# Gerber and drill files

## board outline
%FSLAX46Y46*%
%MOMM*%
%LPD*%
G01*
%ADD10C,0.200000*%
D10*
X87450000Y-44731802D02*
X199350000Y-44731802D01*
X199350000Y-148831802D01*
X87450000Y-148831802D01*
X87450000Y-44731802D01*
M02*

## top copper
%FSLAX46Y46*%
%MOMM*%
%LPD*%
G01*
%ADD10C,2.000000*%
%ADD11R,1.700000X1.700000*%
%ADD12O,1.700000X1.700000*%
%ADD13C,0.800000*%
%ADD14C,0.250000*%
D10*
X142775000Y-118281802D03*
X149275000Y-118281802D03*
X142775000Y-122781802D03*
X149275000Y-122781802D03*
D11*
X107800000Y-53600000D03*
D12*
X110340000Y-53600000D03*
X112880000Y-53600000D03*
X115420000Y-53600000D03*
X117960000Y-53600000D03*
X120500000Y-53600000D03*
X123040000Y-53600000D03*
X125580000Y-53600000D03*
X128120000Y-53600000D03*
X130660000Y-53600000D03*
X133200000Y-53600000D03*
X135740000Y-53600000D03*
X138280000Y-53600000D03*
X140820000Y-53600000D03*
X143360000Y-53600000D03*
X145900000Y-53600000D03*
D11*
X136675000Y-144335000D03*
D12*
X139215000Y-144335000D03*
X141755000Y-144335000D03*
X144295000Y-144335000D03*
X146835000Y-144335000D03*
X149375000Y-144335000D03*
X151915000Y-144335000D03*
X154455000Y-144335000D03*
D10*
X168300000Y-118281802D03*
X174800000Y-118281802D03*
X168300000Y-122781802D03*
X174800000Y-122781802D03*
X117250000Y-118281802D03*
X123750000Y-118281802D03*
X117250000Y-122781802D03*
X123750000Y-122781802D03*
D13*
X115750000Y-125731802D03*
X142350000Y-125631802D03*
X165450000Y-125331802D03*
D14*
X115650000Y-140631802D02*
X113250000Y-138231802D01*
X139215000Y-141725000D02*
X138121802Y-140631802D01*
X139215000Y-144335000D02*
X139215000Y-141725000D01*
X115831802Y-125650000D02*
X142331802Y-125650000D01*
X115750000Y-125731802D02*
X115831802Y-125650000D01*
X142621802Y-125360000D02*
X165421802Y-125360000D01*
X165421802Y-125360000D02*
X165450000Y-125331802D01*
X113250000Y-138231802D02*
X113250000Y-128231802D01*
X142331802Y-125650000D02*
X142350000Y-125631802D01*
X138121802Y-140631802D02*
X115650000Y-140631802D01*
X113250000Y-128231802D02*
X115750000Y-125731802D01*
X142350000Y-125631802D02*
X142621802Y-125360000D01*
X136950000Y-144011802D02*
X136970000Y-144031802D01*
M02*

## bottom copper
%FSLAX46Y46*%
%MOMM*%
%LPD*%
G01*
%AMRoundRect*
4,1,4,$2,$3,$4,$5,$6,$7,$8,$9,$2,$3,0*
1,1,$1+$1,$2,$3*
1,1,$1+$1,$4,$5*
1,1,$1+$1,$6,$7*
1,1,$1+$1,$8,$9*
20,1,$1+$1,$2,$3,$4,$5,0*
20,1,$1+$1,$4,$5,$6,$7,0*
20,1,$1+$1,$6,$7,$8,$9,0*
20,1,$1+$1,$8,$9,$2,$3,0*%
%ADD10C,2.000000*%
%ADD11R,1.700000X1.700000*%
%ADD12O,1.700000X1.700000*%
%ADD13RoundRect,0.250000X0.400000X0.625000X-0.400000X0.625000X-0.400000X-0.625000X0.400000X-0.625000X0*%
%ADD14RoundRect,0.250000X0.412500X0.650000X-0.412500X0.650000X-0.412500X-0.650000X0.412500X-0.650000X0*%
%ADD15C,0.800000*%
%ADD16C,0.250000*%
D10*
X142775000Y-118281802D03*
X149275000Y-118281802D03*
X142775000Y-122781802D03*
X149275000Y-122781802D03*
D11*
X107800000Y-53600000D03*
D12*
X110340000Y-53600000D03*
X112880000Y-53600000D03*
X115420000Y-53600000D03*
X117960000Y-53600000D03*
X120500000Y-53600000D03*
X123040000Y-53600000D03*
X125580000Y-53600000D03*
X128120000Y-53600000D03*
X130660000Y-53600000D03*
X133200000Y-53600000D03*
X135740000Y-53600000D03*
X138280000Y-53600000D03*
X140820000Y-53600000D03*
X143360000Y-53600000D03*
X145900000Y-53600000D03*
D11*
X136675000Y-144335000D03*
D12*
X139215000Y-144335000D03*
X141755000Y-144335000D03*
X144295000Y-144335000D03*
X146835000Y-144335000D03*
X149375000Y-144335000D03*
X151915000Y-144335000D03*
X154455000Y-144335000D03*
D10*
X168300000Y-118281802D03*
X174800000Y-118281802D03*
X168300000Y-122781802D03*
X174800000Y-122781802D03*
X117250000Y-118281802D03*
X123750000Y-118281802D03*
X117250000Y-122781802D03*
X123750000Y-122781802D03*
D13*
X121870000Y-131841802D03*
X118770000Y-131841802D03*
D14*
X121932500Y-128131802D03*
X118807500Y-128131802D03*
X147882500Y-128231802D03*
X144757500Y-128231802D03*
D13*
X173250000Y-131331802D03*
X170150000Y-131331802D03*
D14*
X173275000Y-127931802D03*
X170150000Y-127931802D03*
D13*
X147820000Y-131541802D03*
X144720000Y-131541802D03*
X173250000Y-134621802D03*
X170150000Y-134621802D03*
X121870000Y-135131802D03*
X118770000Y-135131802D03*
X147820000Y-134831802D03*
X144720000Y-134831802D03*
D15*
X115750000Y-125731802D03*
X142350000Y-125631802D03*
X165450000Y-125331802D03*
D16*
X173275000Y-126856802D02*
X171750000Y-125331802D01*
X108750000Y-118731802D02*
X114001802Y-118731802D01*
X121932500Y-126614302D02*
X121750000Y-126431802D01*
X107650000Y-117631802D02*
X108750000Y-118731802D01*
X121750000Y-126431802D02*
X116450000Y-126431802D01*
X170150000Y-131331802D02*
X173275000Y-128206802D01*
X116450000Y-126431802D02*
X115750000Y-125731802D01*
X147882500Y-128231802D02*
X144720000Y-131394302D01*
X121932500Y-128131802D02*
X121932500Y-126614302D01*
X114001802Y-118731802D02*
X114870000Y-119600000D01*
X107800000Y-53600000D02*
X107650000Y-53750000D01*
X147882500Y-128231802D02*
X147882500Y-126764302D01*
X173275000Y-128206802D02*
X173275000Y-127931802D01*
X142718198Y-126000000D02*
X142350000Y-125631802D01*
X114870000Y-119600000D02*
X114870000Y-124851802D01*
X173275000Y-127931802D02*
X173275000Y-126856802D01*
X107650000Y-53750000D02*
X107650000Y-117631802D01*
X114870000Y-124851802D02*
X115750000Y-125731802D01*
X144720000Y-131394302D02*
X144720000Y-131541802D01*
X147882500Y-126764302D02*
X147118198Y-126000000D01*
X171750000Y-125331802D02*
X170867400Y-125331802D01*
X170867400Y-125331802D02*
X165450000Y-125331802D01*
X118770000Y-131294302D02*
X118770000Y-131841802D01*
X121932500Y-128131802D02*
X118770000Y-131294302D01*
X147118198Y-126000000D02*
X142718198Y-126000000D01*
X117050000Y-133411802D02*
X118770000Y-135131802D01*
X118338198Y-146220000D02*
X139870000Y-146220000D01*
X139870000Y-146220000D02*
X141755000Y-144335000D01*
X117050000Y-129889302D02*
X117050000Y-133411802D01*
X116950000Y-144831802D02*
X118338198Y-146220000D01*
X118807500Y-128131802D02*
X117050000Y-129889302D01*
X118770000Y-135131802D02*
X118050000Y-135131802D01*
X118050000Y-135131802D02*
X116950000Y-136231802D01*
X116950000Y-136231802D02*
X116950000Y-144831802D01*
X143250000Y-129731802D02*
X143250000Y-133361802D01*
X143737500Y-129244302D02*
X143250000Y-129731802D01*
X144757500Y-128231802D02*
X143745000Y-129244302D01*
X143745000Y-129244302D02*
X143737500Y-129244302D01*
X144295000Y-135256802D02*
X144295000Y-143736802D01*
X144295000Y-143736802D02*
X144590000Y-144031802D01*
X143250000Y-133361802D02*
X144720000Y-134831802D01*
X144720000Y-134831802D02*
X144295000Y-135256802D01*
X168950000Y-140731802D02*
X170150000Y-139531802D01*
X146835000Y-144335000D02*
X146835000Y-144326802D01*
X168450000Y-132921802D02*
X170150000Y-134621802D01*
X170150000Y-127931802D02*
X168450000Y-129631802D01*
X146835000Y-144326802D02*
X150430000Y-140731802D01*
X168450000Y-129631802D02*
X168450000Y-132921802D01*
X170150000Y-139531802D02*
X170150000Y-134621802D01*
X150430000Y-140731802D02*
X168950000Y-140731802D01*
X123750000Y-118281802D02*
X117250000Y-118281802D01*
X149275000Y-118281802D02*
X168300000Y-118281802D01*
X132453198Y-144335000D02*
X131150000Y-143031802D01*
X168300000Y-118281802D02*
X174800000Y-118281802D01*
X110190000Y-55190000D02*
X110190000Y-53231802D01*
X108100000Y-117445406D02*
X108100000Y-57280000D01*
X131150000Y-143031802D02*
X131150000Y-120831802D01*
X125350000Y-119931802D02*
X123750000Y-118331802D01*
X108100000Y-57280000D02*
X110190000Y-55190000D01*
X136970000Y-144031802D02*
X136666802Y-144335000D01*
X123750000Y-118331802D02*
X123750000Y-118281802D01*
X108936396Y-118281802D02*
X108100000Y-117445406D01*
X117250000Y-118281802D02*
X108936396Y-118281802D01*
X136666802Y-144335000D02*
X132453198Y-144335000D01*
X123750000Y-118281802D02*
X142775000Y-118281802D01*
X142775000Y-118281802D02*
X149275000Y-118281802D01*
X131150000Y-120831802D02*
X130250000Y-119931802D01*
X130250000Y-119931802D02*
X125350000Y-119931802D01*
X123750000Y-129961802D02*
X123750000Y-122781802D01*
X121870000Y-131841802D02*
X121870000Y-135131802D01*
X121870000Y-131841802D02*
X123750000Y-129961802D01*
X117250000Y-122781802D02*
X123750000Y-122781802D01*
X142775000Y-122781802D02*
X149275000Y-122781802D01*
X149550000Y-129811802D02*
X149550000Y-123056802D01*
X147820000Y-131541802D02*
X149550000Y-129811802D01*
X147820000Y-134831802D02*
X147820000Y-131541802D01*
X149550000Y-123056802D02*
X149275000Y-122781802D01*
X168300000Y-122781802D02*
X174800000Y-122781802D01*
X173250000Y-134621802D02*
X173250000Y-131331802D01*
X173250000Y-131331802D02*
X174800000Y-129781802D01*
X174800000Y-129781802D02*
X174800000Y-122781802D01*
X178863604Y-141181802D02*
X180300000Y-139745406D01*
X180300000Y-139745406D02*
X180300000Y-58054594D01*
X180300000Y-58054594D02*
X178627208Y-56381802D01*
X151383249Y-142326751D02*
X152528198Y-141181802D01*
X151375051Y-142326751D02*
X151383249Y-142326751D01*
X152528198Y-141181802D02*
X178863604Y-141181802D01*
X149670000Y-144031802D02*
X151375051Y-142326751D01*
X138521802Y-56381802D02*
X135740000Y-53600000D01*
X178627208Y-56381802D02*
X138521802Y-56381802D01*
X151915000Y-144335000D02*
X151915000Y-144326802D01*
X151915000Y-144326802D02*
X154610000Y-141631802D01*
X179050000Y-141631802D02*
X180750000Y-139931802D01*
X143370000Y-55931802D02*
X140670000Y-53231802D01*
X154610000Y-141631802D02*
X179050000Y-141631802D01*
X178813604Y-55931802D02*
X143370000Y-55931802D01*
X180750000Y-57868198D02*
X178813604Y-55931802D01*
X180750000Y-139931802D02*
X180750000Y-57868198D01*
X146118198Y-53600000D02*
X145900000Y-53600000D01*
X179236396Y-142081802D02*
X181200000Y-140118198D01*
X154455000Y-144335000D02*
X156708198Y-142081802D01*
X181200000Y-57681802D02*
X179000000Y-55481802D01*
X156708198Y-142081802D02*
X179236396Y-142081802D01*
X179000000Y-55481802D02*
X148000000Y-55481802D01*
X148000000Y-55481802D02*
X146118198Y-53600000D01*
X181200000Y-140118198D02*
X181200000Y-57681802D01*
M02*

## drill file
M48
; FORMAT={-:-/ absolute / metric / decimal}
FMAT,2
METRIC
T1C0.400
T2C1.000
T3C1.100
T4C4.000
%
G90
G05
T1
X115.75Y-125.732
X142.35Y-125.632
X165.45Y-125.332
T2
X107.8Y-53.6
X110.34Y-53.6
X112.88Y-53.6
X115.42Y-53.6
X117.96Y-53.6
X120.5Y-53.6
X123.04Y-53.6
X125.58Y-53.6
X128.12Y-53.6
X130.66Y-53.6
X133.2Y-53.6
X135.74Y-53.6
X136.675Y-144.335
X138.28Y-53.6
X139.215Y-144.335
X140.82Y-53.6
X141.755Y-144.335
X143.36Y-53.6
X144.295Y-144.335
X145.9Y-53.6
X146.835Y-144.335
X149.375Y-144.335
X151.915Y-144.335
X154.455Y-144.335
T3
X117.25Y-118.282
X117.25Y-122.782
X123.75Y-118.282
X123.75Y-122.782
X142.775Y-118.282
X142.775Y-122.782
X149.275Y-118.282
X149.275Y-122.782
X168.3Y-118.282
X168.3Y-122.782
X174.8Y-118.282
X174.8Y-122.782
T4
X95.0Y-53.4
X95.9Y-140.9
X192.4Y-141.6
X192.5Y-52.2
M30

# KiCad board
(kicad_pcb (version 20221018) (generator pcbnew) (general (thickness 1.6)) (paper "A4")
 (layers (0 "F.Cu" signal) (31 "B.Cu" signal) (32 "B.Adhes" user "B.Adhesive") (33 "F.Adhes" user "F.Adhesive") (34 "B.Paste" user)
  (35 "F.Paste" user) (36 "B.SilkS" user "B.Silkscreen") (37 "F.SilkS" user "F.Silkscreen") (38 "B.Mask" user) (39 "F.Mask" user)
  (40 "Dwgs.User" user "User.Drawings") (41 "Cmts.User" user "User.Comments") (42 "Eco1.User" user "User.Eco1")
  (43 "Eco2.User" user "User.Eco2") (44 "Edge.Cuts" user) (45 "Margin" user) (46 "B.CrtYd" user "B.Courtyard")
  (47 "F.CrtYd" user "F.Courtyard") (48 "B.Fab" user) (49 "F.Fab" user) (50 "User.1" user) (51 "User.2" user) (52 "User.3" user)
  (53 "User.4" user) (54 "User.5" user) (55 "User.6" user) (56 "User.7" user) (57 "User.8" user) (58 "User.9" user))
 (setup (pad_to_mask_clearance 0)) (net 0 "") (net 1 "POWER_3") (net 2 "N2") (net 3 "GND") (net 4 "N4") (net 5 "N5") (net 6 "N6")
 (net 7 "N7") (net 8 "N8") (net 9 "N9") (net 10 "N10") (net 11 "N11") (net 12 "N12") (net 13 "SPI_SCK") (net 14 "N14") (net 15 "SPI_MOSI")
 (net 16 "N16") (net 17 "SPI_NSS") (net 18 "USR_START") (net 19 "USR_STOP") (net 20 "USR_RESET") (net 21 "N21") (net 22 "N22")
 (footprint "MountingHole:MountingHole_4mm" (layer "F.Cu") (at 192.4 141.6)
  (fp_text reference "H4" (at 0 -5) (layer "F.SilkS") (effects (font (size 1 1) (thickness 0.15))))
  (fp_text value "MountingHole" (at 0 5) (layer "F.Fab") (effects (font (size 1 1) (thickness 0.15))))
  (pad "" np_thru_hole circle (at 0 0) (size 4 4) (drill 4) (layers "*.Cu" "*.Mask")))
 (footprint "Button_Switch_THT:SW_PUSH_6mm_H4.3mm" (layer "F.Cu") (at 142.775 118.281802)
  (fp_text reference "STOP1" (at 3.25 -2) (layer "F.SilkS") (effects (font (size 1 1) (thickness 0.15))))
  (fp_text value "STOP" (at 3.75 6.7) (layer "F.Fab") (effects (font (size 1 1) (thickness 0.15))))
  (pad "1" thru_hole circle (at 0 0 90) (size 2 2) (drill 1.1) (layers "*.Cu" "*.Mask") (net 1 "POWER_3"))
  (pad "1" thru_hole circle (at 6.5 0 90) (size 2 2) (drill 1.1) (layers "*.Cu" "*.Mask") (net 1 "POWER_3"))
  (pad "2" thru_hole circle (at 0 4.5 90) (size 2 2) (drill 1.1) (layers "*.Cu" "*.Mask") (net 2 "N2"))
  (pad "2" thru_hole circle (at 6.5 4.5 90) (size 2 2) (drill 1.1) (layers "*.Cu" "*.Mask") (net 2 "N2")))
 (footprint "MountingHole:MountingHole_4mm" (layer "F.Cu") (at 95.9 140.9)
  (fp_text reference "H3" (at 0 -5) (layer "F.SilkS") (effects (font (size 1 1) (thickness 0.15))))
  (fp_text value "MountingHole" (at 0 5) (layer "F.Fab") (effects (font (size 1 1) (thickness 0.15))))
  (pad "" np_thru_hole circle (at 0 0) (size 4 4) (drill 4) (layers "*.Cu" "*.Mask")))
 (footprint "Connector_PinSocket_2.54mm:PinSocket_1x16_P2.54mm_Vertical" (layer "F.Cu") (at 107.8 53.6 90)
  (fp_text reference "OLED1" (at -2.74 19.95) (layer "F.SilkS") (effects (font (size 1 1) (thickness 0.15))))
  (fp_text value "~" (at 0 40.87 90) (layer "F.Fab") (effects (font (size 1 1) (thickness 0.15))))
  (pad "1" thru_hole rect (at 0 0 90) (size 1.7 1.7) (drill 1) (layers "*.Cu" "*.Mask") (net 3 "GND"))
  (pad "2" thru_hole oval (at 0 2.54 90) (size 1.7 1.7) (drill 1) (layers "*.Cu" "*.Mask") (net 1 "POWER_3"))
  (pad "3" thru_hole oval (at 0 5.08 90) (size 1.7 1.7) (drill 1) (layers "*.Cu" "*.Mask") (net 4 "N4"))
  (pad "4" thru_hole oval (at 0 7.62 90) (size 1.7 1.7) (drill 1) (layers "*.Cu" "*.Mask") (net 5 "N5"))
  (pad "5" thru_hole oval (at 0 10.16 90) (size 1.7 1.7) (drill 1) (layers "*.Cu" "*.Mask") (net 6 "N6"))
  (pad "6" thru_hole oval (at 0 12.7 90) (size 1.7 1.7) (drill 1) (layers "*.Cu" "*.Mask") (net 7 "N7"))
  (pad "7" thru_hole oval (at 0 15.24 90) (size 1.7 1.7) (drill 1) (layers "*.Cu" "*.Mask") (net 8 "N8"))
  (pad "8" thru_hole oval (at 0 17.78 90) (size 1.7 1.7) (drill 1) (layers "*.Cu" "*.Mask") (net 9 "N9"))
  (pad "9" thru_hole oval (at 0 20.32 90) (size 1.7 1.7) (drill 1) (layers "*.Cu" "*.Mask") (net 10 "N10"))
  (pad "10" thru_hole oval (at 0 22.86 90) (size 1.7 1.7) (drill 1) (layers "*.Cu" "*.Mask") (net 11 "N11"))
  (pad "11" thru_hole oval (at 0 25.4 90) (size 1.7 1.7) (drill 1) (layers "*.Cu" "*.Mask") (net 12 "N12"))
  (pad "12" thru_hole oval (at 0 27.94 90) (size 1.7 1.7) (drill 1) (layers "*.Cu" "*.Mask") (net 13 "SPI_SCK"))
  (pad "13" thru_hole oval (at 0 30.48 90) (size 1.7 1.7) (drill 1) (layers "*.Cu" "*.Mask") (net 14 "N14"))
  (pad "14" thru_hole oval (at 0 33.02 90) (size 1.7 1.7) (drill 1) (layers "*.Cu" "*.Mask") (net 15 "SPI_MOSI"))
  (pad "15" thru_hole oval (at 0 35.56 90) (size 1.7 1.7) (drill 1) (layers "*.Cu" "*.Mask") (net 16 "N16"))
  (pad "16" thru_hole oval (at 0 38.1 90) (size 1.7 1.7) (drill 1) (layers "*.Cu" "*.Mask") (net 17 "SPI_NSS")))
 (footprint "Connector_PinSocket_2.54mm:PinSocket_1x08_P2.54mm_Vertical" (layer "F.Cu") (at 136.675 144.335 90)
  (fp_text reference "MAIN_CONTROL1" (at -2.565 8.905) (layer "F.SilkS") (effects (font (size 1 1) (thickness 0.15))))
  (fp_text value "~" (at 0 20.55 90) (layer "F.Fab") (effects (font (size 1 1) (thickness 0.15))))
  (pad "1" thru_hole rect (at 0 0 90) (size 1.7 1.7) (drill 1) (layers "*.Cu" "*.Mask") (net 1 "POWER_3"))
  (pad "2" thru_hole oval (at 0 2.54 90) (size 1.7 1.7) (drill 1) (layers "*.Cu" "*.Mask") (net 3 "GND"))
  (pad "3" thru_hole oval (at 0 5.08 90) (size 1.7 1.7) (drill 1) (layers "*.Cu" "*.Mask") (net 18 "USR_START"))
  (pad "4" thru_hole oval (at 0 7.62 90) (size 1.7 1.7) (drill 1) (layers "*.Cu" "*.Mask") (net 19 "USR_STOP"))
  (pad "5" thru_hole oval (at 0 10.16 90) (size 1.7 1.7) (drill 1) (layers "*.Cu" "*.Mask") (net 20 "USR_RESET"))
  (pad "6" thru_hole oval (at 0 12.7 90) (size 1.7 1.7) (drill 1) (layers "*.Cu" "*.Mask") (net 13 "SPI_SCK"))
  (pad "7" thru_hole oval (at 0 15.24 90) (size 1.7 1.7) (drill 1) (layers "*.Cu" "*.Mask") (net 15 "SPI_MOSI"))
  (pad "8" thru_hole oval (at 0 17.78 90) (size 1.7 1.7) (drill 1) (layers "*.Cu" "*.Mask") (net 17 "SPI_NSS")))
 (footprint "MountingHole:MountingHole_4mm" (layer "F.Cu") (at 192.5 52.2)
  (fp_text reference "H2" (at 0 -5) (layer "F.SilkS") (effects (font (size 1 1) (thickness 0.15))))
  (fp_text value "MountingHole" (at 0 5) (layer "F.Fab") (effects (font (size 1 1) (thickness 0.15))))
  (pad "" np_thru_hole circle (at 0 0) (size 4 4) (drill 4) (layers "*.Cu" "*.Mask")))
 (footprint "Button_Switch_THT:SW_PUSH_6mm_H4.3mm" (layer "F.Cu") (at 168.3 118.281802)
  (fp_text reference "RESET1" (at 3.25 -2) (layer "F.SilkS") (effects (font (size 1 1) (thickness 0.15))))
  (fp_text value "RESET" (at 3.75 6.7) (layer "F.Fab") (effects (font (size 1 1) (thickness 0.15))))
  (pad "1" thru_hole circle (at 0 0 90) (size 2 2) (drill 1.1) (layers "*.Cu" "*.Mask") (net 1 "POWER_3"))
  (pad "1" thru_hole circle (at 6.5 0 90) (size 2 2) (drill 1.1) (layers "*.Cu" "*.Mask") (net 1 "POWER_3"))
  (pad "2" thru_hole circle (at 0 4.5 90) (size 2 2) (drill 1.1) (layers "*.Cu" "*.Mask") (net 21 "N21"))
  (pad "2" thru_hole circle (at 6.5 4.5 90) (size 2 2) (drill 1.1) (layers "*.Cu" "*.Mask") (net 21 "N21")))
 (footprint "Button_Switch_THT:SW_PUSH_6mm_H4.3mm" (layer "F.Cu") (at 117.25 118.281802)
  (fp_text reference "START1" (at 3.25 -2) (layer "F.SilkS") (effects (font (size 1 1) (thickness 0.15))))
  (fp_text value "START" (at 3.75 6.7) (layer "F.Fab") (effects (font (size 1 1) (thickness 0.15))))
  (pad "1" thru_hole circle (at 0 0 90) (size 2 2) (drill 1.1) (layers "*.Cu" "*.Mask") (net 1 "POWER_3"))
  (pad "1" thru_hole circle (at 6.5 0 90) (size 2 2) (drill 1.1) (layers "*.Cu" "*.Mask") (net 1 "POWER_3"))
  (pad "2" thru_hole circle (at 0 4.5 90) (size 2 2) (drill 1.1) (layers "*.Cu" "*.Mask") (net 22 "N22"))
  (pad "2" thru_hole circle (at 6.5 4.5 90) (size 2 2) (drill 1.1) (layers "*.Cu" "*.Mask") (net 22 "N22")))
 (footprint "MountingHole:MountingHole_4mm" (layer "F.Cu") (at 95 53.4)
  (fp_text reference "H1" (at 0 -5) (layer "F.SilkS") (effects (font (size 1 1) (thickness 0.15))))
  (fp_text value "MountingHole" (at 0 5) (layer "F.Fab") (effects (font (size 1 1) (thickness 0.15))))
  (pad "" np_thru_hole circle (at 0 0) (size 4 4) (drill 4) (layers "*.Cu" "*.Mask")))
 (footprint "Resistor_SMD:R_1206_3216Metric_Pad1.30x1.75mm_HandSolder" (layer "B.Cu") (at 120.32 131.841802 180)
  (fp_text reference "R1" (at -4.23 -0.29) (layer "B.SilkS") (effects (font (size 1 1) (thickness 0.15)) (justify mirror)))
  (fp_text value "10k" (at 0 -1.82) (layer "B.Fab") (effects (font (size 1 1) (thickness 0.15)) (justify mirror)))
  (pad "1" smd roundrect (at -1.55 0 180) (size 1.3 1.75) (layers "B.Cu" "B.Paste" "B.Mask") (roundrect_rratio 0.192308) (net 22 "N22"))
  (pad "2" smd roundrect (at 1.55 0 180) (size 1.3 1.75) (layers "B.Cu" "B.Paste" "B.Mask") (roundrect_rratio 0.192308) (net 3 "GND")))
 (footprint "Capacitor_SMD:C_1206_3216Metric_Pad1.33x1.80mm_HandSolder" (layer "B.Cu") (at 120.37 128.131802 180)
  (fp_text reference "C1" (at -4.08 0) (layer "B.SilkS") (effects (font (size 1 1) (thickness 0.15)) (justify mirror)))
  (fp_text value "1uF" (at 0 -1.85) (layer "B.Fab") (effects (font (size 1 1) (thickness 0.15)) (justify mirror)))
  (pad "1" smd roundrect (at -1.5625 0 180) (size 1.325 1.8) (layers "B.Cu" "B.Paste" "B.Mask") (roundrect_rratio 0.188679) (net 3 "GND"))
  (pad "2" smd roundrect (at 1.5625 0 180) (size 1.325 1.8) (layers "B.Cu" "B.Paste" "B.Mask") (roundrect_rratio 0.188679)
   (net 18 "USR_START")))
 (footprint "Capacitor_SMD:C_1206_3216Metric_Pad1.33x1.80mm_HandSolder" (layer "B.Cu") (at 146.32 128.231802 180)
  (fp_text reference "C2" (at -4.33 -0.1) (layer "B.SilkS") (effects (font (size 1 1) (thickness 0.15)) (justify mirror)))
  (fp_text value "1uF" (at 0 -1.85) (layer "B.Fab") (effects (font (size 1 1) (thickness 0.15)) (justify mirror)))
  (pad "1" smd roundrect (at -1.5625 0 180) (size 1.325 1.8) (layers "B.Cu" "B.Paste" "B.Mask") (roundrect_rratio 0.188679) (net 3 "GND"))
  (pad "2" smd roundrect (at 1.5625 0 180) (size 1.325 1.8) (layers "B.Cu" "B.Paste" "B.Mask") (roundrect_rratio 0.188679)
   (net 19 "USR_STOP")))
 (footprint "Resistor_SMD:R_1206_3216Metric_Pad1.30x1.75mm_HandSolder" (layer "B.Cu") (at 171.7 131.331802 180)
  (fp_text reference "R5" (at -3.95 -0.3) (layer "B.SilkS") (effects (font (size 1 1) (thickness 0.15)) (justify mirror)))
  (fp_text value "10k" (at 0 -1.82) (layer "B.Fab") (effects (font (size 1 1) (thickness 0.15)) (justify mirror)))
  (pad "1" smd roundrect (at -1.55 0 180) (size 1.3 1.75) (layers "B.Cu" "B.Paste" "B.Mask") (roundrect_rratio 0.192308) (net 21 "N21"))
  (pad "2" smd roundrect (at 1.55 0 180) (size 1.3 1.75) (layers "B.Cu" "B.Paste" "B.Mask") (roundrect_rratio 0.192308) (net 3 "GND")))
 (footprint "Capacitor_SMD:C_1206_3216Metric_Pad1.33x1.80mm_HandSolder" (layer "B.Cu") (at 171.7125 127.931802 180)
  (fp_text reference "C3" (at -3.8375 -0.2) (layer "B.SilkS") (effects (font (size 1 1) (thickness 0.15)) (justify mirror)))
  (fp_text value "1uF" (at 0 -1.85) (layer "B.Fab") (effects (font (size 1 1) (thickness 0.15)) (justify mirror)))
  (pad "1" smd roundrect (at -1.5625 0 180) (size 1.325 1.8) (layers "B.Cu" "B.Paste" "B.Mask") (roundrect_rratio 0.188679) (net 3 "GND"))
  (pad "2" smd roundrect (at 1.5625 0 180) (size 1.325 1.8) (layers "B.Cu" "B.Paste" "B.Mask") (roundrect_rratio 0.188679)
   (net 20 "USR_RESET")))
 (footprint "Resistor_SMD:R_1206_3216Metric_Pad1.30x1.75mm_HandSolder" (layer "B.Cu") (at 146.27 131.541802 180)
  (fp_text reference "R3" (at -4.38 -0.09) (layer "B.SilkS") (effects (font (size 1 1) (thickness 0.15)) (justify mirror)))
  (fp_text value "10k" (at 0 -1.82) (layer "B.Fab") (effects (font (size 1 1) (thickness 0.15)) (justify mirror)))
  (pad "1" smd roundrect (at -1.55 0 180) (size 1.3 1.75) (layers "B.Cu" "B.Paste" "B.Mask") (roundrect_rratio 0.192308) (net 2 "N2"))
  (pad "2" smd roundrect (at 1.55 0 180) (size 1.3 1.75) (layers "B.Cu" "B.Paste" "B.Mask") (roundrect_rratio 0.192308) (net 3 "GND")))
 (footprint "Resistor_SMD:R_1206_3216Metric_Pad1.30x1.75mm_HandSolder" (layer "B.Cu") (at 171.7 134.621802 180)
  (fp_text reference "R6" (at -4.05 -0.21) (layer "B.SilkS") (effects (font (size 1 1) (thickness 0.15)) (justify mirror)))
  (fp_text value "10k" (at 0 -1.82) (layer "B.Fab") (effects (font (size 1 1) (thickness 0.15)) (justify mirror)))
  (pad "1" smd roundrect (at -1.55 0 180) (size 1.3 1.75) (layers "B.Cu" "B.Paste" "B.Mask") (roundrect_rratio 0.192308) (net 21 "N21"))
  (pad "2" smd roundrect (at 1.55 0 180) (size 1.3 1.75) (layers "B.Cu" "B.Paste" "B.Mask") (roundrect_rratio 0.192308) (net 20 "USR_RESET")))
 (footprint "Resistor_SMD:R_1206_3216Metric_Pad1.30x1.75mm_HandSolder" (layer "B.Cu") (at 120.32 135.131802 180)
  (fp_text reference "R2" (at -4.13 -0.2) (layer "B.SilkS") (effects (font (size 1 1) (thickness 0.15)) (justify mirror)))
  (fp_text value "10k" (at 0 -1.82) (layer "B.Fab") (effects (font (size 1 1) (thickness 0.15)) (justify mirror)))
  (pad "1" smd roundrect (at -1.55 0 180) (size 1.3 1.75) (layers "B.Cu" "B.Paste" "B.Mask") (roundrect_rratio 0.192308) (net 22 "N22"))
  (pad "2" smd roundrect (at 1.55 0 180) (size 1.3 1.75) (layers "B.Cu" "B.Paste" "B.Mask") (roundrect_rratio 0.192308) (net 18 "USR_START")))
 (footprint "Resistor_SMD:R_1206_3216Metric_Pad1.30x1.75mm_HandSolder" (layer "B.Cu") (at 146.27 134.831802 180)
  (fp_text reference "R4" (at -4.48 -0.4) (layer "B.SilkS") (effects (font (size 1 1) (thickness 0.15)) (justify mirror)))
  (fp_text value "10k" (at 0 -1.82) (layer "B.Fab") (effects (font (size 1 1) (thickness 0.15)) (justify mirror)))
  (pad "1" smd roundrect (at -1.55 0 180) (size 1.3 1.75) (layers "B.Cu" "B.Paste" "B.Mask") (roundrect_rratio 0.192308) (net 2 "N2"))
  (pad "2" smd roundrect (at 1.55 0 180) (size 1.3 1.75) (layers "B.Cu" "B.Paste" "B.Mask") (roundrect_rratio 0.192308) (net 19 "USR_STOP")))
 (gr_rect (start 87.45 44.731802) (end 199.35 148.831802) (stroke (width 0.2) (type default)) (fill none) (layer "Edge.Cuts"))
 (segment (start 115.65 140.631802) (end 113.25 138.231802) (width 0.25) (layer "F.Cu") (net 3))
 (segment (start 139.215 141.725) (end 138.121802 140.631802) (width 0.25) (layer "F.Cu") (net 3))
 (segment (start 139.215 144.335) (end 139.215 141.725) (width 0.25) (layer "F.Cu") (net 3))
 (segment (start 115.831802 125.65) (end 142.331802 125.65) (width 0.25) (layer "F.Cu") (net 3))
 (segment (start 115.75 125.731802) (end 115.831802 125.65) (width 0.25) (layer "F.Cu") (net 3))
 (segment (start 142.621802 125.36) (end 165.421802 125.36) (width 0.25) (layer "F.Cu") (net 3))
 (segment (start 165.421802 125.36) (end 165.45 125.331802) (width 0.25) (layer "F.Cu") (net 3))
 (segment (start 113.25 138.231802) (end 113.25 128.231802) (width 0.25) (layer "F.Cu") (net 3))
 (segment (start 142.331802 125.65) (end 142.35 125.631802) (width 0.25) (layer "F.Cu") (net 3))
 (segment (start 138.121802 140.631802) (end 115.65 140.631802) (width 0.25) (layer "F.Cu") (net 3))
 (segment (start 113.25 128.231802) (end 115.75 125.731802) (width 0.25) (layer "F.Cu") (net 3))
 (segment (start 142.35 125.631802) (end 142.621802 125.36) (width 0.25) (layer "F.Cu") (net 3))
 (via (at 115.75 125.731802) (size 0.8) (drill 0.4) (layers "F.Cu" "B.Cu") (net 3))
 (via (at 142.35 125.631802) (size 0.8) (drill 0.4) (layers "F.Cu" "B.Cu") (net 3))
 (via (at 165.45 125.331802) (size 0.8) (drill 0.4) (layers "F.Cu" "B.Cu") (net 3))
 (segment (start 173.275 126.856802) (end 171.75 125.331802) (width 0.25) (layer "B.Cu") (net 3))
 (segment (start 108.75 118.731802) (end 114.001802 118.731802) (width 0.25) (layer "B.Cu") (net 3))
 (segment (start 121.9325 126.614302) (end 121.75 126.431802) (width 0.25) (layer "B.Cu") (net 3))
 (segment (start 107.65 117.631802) (end 108.75 118.731802) (width 0.25) (layer "B.Cu") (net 3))
 (segment (start 121.75 126.431802) (end 116.45 126.431802) (width 0.25) (layer "B.Cu") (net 3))
 (segment (start 170.15 131.331802) (end 173.275 128.206802) (width 0.25) (layer "B.Cu") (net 3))
 (segment (start 116.45 126.431802) (end 115.75 125.731802) (width 0.25) (layer "B.Cu") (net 3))
 (segment (start 147.8825 128.231802) (end 144.72 131.394302) (width 0.25) (layer "B.Cu") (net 3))
 (segment (start 121.9325 128.131802) (end 121.9325 126.614302) (width 0.25) (layer "B.Cu") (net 3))
 (segment (start 114.001802 118.731802) (end 114.87 119.6) (width 0.25) (layer "B.Cu") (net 3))
 (segment (start 107.8 53.6) (end 107.65 53.75) (width 0.25) (layer "B.Cu") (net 3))
 (segment (start 147.8825 128.231802) (end 147.8825 126.764302) (width 0.25) (layer "B.Cu") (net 3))
 (segment (start 173.275 128.206802) (end 173.275 127.931802) (width 0.25) (layer "B.Cu") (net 3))
 (segment (start 142.718198 126) (end 142.35 125.631802) (width 0.25) (layer "B.Cu") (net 3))
 (segment (start 114.87 119.6) (end 114.87 124.851802) (width 0.25) (layer "B.Cu") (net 3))
 (segment (start 173.275 127.931802) (end 173.275 126.856802) (width 0.25) (layer "B.Cu") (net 3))
 (segment (start 107.65 53.75) (end 107.65 117.631802) (width 0.25) (layer "B.Cu") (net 3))
 (segment (start 114.87 124.851802) (end 115.75 125.731802) (width 0.25) (layer "B.Cu") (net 3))
 (segment (start 144.72 131.394302) (end 144.72 131.541802) (width 0.25) (layer "B.Cu") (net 3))
 (segment (start 147.8825 126.764302) (end 147.118198 126) (width 0.25) (layer "B.Cu") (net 3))
 (segment (start 171.75 125.331802) (end 170.8674 125.331802) (width 0.25) (layer "B.Cu") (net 3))
 (segment (start 170.8674 125.331802) (end 165.45 125.331802) (width 0.25) (layer "B.Cu") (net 3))
 (segment (start 118.77 131.294302) (end 118.77 131.841802) (width 0.25) (layer "B.Cu") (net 3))
 (segment (start 121.9325 128.131802) (end 118.77 131.294302) (width 0.25) (layer "B.Cu") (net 3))
 (segment (start 147.118198 126) (end 142.718198 126) (width 0.25) (layer "B.Cu") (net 3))
 (segment (start 117.05 133.411802) (end 118.77 135.131802) (width 0.25) (layer "B.Cu") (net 18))
 (segment (start 118.338198 146.22) (end 139.87 146.22) (width 0.25) (layer "B.Cu") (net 18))
 (segment (start 139.87 146.22) (end 141.755 144.335) (width 0.25) (layer "B.Cu") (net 18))
 (segment (start 117.05 129.889302) (end 117.05 133.411802) (width 0.25) (layer "B.Cu") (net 18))
 (segment (start 116.95 144.831802) (end 118.338198 146.22) (width 0.25) (layer "B.Cu") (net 18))
 (segment (start 118.8075 128.131802) (end 117.05 129.889302) (width 0.25) (layer "B.Cu") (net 18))
 (segment (start 118.77 135.131802) (end 118.05 135.131802) (width 0.25) (layer "B.Cu") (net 18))
 (segment (start 118.05 135.131802) (end 116.95 136.231802) (width 0.25) (layer "B.Cu") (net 18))
 (segment (start 116.95 136.231802) (end 116.95 144.831802) (width 0.25) (layer "B.Cu") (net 18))
 (segment (start 143.25 129.731802) (end 143.25 133.361802) (width 0.25) (layer "B.Cu") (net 19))
 (segment (start 143.7375 129.244302) (end 143.25 129.731802) (width 0.25) (layer "B.Cu") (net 19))
 (segment (start 144.7575 128.231802) (end 143.745 129.244302) (width 0.25) (layer "B.Cu") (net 19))
 (segment (start 143.745 129.244302) (end 143.7375 129.244302) (width 0.25) (layer "B.Cu") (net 19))
 (segment (start 144.295 135.256802) (end 144.295 143.736802) (width 0.25) (layer "B.Cu") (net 19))
 (segment (start 144.295 143.736802) (end 144.59 144.031802) (width 0.25) (layer "B.Cu") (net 19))
 (segment (start 143.25 133.361802) (end 144.72 134.831802) (width 0.25) (layer "B.Cu") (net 19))
 (segment (start 144.72 134.831802) (end 144.295 135.256802) (width 0.25) (layer "B.Cu") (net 19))
 (segment (start 168.95 140.731802) (end 170.15 139.531802) (width 0.25) (layer "B.Cu") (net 20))
 (segment (start 146.835 144.335) (end 146.835 144.326802) (width 0.25) (layer "B.Cu") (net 20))
 (segment (start 168.45 132.921802) (end 170.15 134.621802) (width 0.25) (layer "B.Cu") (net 20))
 (segment (start 170.15 127.931802) (end 168.45 129.631802) (width 0.25) (layer "B.Cu") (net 20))
 (segment (start 146.835 144.326802) (end 150.43 140.731802) (width 0.25) (layer "B.Cu") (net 20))
 (segment (start 168.45 129.631802) (end 168.45 132.921802) (width 0.25) (layer "B.Cu") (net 20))
 (segment (start 170.15 139.531802) (end 170.15 134.621802) (width 0.25) (layer "B.Cu") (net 20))
 (segment (start 150.43 140.731802) (end 168.95 140.731802) (width 0.25) (layer "B.Cu") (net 20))
 (segment (start 136.95 144.011802) (end 136.97 144.031802) (width 0.25) (layer "F.Cu") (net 1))
 (segment (start 123.75 118.281802) (end 117.25 118.281802) (width 0.25) (layer "B.Cu") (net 1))
 (segment (start 149.275 118.281802) (end 168.3 118.281802) (width 0.25) (layer "B.Cu") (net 1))
 (segment (start 132.453198 144.335) (end 131.15 143.031802) (width 0.25) (layer "B.Cu") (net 1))
 (segment (start 168.3 118.281802) (end 174.8 118.281802) (width 0.25) (layer "B.Cu") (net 1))
 (segment (start 110.19 55.19) (end 110.19 53.231802) (width 0.25) (layer "B.Cu") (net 1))
 (segment (start 108.1 117.445406) (end 108.1 57.28) (width 0.25) (layer "B.Cu") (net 1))
 (segment (start 131.15 143.031802) (end 131.15 120.831802) (width 0.25) (layer "B.Cu") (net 1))
 (segment (start 125.35 119.931802) (end 123.75 118.331802) (width 0.25) (layer "B.Cu") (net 1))
 (segment (start 108.1 57.28) (end 110.19 55.19) (width 0.25) (layer "B.Cu") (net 1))
 (segment (start 136.97 144.031802) (end 136.666802 144.335) (width 0.25) (layer "B.Cu") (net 1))
 (segment (start 123.75 118.331802) (end 123.75 118.281802) (width 0.25) (layer "B.Cu") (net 1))
 (segment (start 108.936396 118.281802) (end 108.1 117.445406) (width 0.25) (layer "B.Cu") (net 1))
 (segment (start 117.25 118.281802) (end 108.936396 118.281802) (width 0.25) (layer "B.Cu") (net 1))
 (segment (start 136.666802 144.335) (end 132.453198 144.335) (width 0.25) (layer "B.Cu") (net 1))
 (segment (start 123.75 118.281802) (end 142.775 118.281802) (width 0.25) (layer "B.Cu") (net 1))
 (segment (start 142.775 118.281802) (end 149.275 118.281802) (width 0.25) (layer "B.Cu") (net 1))
 (segment (start 131.15 120.831802) (end 130.25 119.931802) (width 0.25) (layer "B.Cu") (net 1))
 (segment (start 130.25 119.931802) (end 125.35 119.931802) (width 0.25) (layer "B.Cu") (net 1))
 (segment (start 123.75 129.961802) (end 123.75 122.781802) (width 0.25) (layer "B.Cu") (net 22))
 (segment (start 121.87 131.841802) (end 121.87 135.131802) (width 0.25) (layer "B.Cu") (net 22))
 (segment (start 121.87 131.841802) (end 123.75 129.961802) (width 0.25) (layer "B.Cu") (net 22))
 (segment (start 117.25 122.781802) (end 123.75 122.781802) (width 0.25) (layer "B.Cu") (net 22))
 (segment (start 142.775 122.781802) (end 149.275 122.781802) (width 0.25) (layer "B.Cu") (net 2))
 (segment (start 149.55 129.811802) (end 149.55 123.056802) (width 0.25) (layer "B.Cu") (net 2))
 (segment (start 147.82 131.541802) (end 149.55 129.811802) (width 0.25) (layer "B.Cu") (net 2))
 (segment (start 147.82 134.831802) (end 147.82 131.541802) (width 0.25) (layer "B.Cu") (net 2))
 (segment (start 149.55 123.056802) (end 149.275 122.781802) (width 0.25) (layer "B.Cu") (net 2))
 (segment (start 168.3 122.781802) (end 174.8 122.781802) (width 0.25) (layer "B.Cu") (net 21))
 (segment (start 173.25 134.621802) (end 173.25 131.331802) (width 0.25) (layer "B.Cu") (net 21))
 (segment (start 173.25 131.331802) (end 174.8 129.781802) (width 0.25) (layer "B.Cu") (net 21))
 (segment (start 174.8 129.781802) (end 174.8 122.781802) (width 0.25) (layer "B.Cu") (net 21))
 (segment (start 178.863604 141.181802) (end 180.3 139.745406) (width 0.25) (layer "B.Cu") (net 13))
 (segment (start 180.3 139.745406) (end 180.3 58.054594) (width 0.25) (layer "B.Cu") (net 13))
 (segment (start 180.3 58.054594) (end 178.627208 56.381802) (width 0.25) (layer "B.Cu") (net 13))
 (segment (start 151.383249 142.326751) (end 152.528198 141.181802) (width 0.25) (layer "B.Cu") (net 13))
 (segment (start 151.375051 142.326751) (end 151.383249 142.326751) (width 0.25) (layer "B.Cu") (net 13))
 (segment (start 152.528198 141.181802) (end 178.863604 141.181802) (width 0.25) (layer "B.Cu") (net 13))
 (segment (start 149.67 144.031802) (end 151.375051 142.326751) (width 0.25) (layer "B.Cu") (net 13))
 (segment (start 138.521802 56.381802) (end 135.74 53.6) (width 0.25) (layer "B.Cu") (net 13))
 (segment (start 178.627208 56.381802) (end 138.521802 56.381802) (width 0.25) (layer "B.Cu") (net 13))
 (segment (start 151.915 144.335) (end 151.915 144.326802) (width 0.25) (layer "B.Cu") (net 15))
 (segment (start 151.915 144.326802) (end 154.61 141.631802) (width 0.25) (layer "B.Cu") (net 15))
 (segment (start 179.05 141.631802) (end 180.75 139.931802) (width 0.25) (layer "B.Cu") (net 15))
 (segment (start 143.37 55.931802) (end 140.67 53.231802) (width 0.25) (layer "B.Cu") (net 15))
 (segment (start 154.61 141.631802) (end 179.05 141.631802) (width 0.25) (layer "B.Cu") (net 15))
 (segment (start 178.813604 55.931802) (end 143.37 55.931802) (width 0.25) (layer "B.Cu") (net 15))
 (segment (start 180.75 57.868198) (end 178.813604 55.931802) (width 0.25) (layer "B.Cu") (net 15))
 (segment (start 180.75 139.931802) (end 180.75 57.868198) (width 0.25) (layer "B.Cu") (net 15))
 (segment (start 146.118198 53.6) (end 145.9 53.6) (width 0.25) (layer "B.Cu") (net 17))
 (segment (start 179.236396 142.081802) (end 181.2 140.118198) (width 0.25) (layer "B.Cu") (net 17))
 (segment (start 154.455 144.335) (end 156.708198 142.081802) (width 0.25) (layer "B.Cu") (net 17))
 (segment (start 181.2 57.681802) (end 179 55.481802) (width 0.25) (layer "B.Cu") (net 17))
 (segment (start 156.708198 142.081802) (end 179.236396 142.081802) (width 0.25) (layer "B.Cu") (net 17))
 (segment (start 179 55.481802) (end 148 55.481802) (width 0.25) (layer "B.Cu") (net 17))
 (segment (start 148 55.481802) (end 146.118198 53.6) (width 0.25) (layer "B.Cu") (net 17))
 (segment (start 181.2 140.118198) (end 181.2 57.681802) (width 0.25) (layer "B.Cu") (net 17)))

